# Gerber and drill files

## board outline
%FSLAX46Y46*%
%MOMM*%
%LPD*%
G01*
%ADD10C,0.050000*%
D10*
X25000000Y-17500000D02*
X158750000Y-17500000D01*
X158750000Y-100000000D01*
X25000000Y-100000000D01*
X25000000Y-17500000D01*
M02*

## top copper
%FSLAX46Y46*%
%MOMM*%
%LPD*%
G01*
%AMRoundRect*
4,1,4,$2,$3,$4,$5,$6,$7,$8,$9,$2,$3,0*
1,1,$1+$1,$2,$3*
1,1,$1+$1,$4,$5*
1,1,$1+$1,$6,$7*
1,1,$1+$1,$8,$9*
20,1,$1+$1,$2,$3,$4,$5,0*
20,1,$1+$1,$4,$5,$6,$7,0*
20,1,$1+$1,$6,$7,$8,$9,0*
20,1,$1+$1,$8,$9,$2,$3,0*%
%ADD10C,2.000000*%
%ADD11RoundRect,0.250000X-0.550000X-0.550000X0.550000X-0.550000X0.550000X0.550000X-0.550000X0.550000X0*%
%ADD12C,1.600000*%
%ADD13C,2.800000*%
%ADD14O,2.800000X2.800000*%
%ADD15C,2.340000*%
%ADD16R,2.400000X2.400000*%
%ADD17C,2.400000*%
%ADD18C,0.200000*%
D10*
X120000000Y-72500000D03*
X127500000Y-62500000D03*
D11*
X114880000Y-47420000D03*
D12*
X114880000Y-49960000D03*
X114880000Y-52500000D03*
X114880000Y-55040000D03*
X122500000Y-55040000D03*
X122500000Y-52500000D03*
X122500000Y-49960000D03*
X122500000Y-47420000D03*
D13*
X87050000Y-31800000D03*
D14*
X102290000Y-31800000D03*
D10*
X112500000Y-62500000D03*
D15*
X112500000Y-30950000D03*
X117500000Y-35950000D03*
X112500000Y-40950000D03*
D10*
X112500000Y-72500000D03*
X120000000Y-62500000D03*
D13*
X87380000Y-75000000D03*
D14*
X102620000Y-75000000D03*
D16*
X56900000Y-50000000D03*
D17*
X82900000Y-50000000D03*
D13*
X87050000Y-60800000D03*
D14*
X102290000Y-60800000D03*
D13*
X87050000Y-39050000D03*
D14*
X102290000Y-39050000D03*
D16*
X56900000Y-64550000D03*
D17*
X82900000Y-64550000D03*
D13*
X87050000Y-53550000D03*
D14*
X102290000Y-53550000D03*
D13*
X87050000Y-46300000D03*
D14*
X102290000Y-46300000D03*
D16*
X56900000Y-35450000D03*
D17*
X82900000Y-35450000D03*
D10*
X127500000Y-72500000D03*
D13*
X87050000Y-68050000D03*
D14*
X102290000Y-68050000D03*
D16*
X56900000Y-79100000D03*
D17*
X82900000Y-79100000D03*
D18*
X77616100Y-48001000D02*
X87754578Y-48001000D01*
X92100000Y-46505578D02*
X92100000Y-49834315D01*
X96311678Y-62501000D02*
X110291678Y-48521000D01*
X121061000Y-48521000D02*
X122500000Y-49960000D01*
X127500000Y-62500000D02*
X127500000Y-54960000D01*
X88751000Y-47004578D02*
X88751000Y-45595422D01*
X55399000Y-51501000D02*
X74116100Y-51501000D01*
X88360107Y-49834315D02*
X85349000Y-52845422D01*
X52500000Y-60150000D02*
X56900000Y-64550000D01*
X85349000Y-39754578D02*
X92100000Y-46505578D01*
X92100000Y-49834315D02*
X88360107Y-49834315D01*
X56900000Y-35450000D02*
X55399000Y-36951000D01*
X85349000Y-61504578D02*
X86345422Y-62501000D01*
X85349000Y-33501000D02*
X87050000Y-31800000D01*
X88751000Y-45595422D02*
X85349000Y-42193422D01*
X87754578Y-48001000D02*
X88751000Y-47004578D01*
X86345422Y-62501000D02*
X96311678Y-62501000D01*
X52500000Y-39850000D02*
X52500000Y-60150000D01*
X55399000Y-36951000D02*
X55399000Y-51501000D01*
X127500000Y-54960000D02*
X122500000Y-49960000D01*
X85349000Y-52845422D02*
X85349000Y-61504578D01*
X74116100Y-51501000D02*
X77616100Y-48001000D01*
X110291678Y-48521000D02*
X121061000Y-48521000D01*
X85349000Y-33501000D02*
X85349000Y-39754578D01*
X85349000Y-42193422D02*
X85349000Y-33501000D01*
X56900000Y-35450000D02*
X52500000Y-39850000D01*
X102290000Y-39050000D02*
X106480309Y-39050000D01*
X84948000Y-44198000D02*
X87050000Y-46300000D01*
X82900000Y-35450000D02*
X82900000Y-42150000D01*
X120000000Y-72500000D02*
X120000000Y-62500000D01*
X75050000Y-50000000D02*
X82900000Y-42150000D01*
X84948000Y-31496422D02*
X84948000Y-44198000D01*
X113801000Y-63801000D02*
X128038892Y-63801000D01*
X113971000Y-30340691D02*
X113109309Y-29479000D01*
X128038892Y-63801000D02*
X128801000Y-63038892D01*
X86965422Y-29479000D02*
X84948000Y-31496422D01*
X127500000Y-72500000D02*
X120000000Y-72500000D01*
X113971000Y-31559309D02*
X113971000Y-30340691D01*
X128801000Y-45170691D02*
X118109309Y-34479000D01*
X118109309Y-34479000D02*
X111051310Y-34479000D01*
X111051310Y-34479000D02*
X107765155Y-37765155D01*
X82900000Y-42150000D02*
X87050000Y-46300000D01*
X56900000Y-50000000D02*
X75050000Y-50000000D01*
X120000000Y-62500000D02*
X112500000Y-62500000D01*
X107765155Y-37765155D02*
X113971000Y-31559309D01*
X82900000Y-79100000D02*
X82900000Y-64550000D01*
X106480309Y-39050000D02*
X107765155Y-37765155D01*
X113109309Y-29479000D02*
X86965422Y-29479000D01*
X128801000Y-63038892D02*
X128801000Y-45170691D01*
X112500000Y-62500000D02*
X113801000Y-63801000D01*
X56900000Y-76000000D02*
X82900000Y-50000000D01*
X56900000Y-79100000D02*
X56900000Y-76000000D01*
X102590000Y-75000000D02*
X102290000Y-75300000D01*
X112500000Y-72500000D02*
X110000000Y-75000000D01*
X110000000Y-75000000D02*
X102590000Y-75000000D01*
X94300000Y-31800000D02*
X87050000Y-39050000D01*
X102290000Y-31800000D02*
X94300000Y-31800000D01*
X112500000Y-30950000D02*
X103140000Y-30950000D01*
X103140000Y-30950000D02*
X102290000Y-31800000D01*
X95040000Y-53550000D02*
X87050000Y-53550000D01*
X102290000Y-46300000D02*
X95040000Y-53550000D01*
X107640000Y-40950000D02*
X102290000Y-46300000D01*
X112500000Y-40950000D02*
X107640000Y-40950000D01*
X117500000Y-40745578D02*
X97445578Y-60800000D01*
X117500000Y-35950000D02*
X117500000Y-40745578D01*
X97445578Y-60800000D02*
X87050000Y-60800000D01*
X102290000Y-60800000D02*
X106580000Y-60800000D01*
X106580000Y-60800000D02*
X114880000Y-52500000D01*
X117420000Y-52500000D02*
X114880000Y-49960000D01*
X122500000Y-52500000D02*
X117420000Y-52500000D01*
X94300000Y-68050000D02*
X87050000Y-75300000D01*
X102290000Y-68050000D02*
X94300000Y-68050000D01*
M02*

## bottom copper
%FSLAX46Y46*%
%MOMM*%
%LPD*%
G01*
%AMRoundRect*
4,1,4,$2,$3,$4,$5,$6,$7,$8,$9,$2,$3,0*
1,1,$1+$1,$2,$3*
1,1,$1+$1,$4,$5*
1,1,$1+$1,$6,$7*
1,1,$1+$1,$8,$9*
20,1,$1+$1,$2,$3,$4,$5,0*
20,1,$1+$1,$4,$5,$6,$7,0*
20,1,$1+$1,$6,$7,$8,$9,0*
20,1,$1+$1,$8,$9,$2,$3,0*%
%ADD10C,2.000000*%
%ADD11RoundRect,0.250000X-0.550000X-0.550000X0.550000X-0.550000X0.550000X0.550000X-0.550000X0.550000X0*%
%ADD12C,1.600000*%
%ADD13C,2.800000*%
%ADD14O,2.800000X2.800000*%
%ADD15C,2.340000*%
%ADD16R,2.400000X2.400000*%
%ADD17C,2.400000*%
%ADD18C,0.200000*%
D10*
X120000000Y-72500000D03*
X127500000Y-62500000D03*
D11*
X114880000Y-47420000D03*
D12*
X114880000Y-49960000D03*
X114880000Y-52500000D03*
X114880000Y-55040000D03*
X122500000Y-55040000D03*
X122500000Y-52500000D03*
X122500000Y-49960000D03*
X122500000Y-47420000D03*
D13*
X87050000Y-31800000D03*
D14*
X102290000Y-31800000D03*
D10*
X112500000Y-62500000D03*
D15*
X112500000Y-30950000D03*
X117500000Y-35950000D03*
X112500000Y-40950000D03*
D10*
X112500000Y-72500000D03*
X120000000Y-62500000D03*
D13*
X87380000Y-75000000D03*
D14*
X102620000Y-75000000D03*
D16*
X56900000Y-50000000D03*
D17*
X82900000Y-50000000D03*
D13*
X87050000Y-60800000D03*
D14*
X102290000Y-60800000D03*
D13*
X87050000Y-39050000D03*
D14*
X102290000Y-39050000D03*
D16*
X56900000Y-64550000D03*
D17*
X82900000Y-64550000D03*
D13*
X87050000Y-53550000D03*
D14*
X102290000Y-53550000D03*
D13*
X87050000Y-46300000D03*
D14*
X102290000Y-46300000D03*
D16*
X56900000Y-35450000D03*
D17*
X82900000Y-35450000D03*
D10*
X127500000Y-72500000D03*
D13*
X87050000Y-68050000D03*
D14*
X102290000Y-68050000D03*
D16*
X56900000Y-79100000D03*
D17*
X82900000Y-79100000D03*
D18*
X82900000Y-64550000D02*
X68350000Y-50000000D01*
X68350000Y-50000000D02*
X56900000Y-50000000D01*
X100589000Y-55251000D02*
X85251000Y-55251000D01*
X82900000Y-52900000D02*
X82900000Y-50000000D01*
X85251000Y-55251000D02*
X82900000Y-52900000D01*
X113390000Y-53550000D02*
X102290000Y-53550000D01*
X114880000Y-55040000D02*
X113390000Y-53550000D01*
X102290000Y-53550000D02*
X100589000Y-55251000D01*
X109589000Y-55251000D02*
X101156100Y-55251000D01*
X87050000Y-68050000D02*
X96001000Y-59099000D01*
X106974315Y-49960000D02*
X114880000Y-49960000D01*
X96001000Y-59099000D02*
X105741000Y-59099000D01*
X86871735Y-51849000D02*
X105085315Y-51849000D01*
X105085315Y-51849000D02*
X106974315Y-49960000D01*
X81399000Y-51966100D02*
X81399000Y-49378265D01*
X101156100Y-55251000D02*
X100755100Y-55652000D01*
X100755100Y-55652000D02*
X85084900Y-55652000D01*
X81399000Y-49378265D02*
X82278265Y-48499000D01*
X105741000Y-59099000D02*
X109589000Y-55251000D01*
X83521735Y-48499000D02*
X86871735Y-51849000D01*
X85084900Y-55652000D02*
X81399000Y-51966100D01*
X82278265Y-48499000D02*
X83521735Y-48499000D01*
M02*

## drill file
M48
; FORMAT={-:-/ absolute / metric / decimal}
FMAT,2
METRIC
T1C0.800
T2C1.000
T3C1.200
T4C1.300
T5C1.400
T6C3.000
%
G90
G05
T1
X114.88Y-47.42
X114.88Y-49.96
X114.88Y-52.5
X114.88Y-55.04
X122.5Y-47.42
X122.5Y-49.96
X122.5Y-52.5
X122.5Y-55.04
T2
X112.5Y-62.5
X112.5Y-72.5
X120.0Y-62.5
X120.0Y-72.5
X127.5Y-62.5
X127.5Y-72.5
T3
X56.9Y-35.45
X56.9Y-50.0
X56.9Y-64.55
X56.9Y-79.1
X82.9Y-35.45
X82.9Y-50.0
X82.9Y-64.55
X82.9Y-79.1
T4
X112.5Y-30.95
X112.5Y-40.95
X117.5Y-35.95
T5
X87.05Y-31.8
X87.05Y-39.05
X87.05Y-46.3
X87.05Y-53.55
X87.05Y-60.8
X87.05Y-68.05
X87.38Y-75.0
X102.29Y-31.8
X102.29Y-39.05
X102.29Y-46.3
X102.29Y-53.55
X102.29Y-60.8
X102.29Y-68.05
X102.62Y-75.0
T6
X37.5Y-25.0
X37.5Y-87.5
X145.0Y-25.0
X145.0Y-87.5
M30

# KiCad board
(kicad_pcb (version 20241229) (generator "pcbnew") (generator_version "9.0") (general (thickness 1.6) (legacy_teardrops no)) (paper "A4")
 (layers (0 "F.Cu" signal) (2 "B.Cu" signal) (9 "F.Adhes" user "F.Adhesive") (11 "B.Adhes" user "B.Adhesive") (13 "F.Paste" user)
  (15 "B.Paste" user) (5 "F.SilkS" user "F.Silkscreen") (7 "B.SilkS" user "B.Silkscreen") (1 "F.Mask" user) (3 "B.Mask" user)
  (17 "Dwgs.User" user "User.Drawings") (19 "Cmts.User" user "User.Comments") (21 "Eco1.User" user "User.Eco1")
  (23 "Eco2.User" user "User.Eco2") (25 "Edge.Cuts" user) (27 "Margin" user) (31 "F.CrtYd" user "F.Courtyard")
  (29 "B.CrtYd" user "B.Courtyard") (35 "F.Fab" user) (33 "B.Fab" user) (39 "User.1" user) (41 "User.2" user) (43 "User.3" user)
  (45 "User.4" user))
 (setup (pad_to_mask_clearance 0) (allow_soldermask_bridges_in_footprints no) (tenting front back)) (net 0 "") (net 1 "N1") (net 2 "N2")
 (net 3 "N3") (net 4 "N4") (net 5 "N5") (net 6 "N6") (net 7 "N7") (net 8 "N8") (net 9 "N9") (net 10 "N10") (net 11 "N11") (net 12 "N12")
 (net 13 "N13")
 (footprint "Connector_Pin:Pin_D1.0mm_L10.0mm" (layer "F.Cu") (at 120 72.5)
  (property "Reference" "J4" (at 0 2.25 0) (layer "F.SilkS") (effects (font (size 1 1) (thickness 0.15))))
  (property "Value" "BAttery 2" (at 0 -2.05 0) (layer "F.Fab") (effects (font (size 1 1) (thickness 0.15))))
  (pad "1" thru_hole circle (at 0 0) (size 2 2) (drill 1) (layers "*.Cu" "*.Mask") (remove_unused_layers no) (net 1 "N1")))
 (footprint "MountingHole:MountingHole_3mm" (layer "F.Cu") (at 145 25)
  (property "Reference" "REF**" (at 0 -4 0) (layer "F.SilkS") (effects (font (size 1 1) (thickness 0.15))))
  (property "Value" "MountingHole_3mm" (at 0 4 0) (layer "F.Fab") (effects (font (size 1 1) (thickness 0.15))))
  (pad "" np_thru_hole circle (at 0 0) (size 3 3) (drill 3) (layers "*.Cu" "*.Mask")))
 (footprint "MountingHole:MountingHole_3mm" (layer "F.Cu") (at 37.5 25)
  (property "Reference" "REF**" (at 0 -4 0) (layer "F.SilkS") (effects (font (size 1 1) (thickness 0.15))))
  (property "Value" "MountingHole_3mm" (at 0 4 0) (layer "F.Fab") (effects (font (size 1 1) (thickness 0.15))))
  (pad "" np_thru_hole circle (at 0 0) (size 3 3) (drill 3) (layers "*.Cu" "*.Mask")))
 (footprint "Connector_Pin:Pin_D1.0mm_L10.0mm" (layer "F.Cu") (at 127.5 62.5)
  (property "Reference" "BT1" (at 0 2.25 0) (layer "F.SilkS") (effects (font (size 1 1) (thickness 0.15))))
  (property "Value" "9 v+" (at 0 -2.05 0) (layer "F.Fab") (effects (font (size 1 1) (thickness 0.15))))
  (pad "1" thru_hole circle (at 0 0) (size 2 2) (drill 1) (layers "*.Cu" "*.Mask") (remove_unused_layers no) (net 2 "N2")))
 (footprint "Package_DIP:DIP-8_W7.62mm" (layer "F.Cu") (at 114.88 47.42)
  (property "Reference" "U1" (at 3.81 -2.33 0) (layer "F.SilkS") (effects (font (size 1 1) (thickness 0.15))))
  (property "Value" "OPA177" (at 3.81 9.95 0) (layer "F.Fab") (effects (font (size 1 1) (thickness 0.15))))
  (pad "1" thru_hole roundrect (at 0 0) (size 1.6 1.6) (drill 0.8) (layers "*.Cu" "*.Mask") (remove_unused_layers no)
   (roundrect_rratio 0.15625) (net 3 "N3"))
  (pad "2" thru_hole circle (at 0 2.54) (size 1.6 1.6) (drill 0.8) (layers "*.Cu" "*.Mask") (remove_unused_layers no) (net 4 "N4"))
  (pad "3" thru_hole circle (at 0 5.08) (size 1.6 1.6) (drill 0.8) (layers "*.Cu" "*.Mask") (remove_unused_layers no) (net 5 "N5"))
  (pad "4" thru_hole circle (at 0 7.62) (size 1.6 1.6) (drill 0.8) (layers "*.Cu" "*.Mask") (remove_unused_layers no) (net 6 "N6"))
  (pad "5" thru_hole circle (at 7.62 7.62) (size 1.6 1.6) (drill 0.8) (layers "*.Cu" "*.Mask") (remove_unused_layers no) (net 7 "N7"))
  (pad "6" thru_hole circle (at 7.62 5.08) (size 1.6 1.6) (drill 0.8) (layers "*.Cu" "*.Mask") (remove_unused_layers no) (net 4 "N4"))
  (pad "7" thru_hole circle (at 7.62 2.54) (size 1.6 1.6) (drill 0.8) (layers "*.Cu" "*.Mask") (remove_unused_layers no) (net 2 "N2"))
  (pad "8" thru_hole circle (at 7.62 0) (size 1.6 1.6) (drill 0.8) (layers "*.Cu" "*.Mask") (remove_unused_layers no) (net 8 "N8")))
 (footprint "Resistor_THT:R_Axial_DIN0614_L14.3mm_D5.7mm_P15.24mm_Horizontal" (layer "F.Cu") (at 87.05 31.8)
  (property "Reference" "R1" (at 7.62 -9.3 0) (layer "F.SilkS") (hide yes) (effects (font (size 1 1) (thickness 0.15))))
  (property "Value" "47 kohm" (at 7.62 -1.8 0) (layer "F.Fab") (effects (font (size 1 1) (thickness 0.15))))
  (pad "1" thru_hole circle (at 0 0) (size 2.8 2.8) (drill 1.4) (layers "*.Cu" "*.Mask") (remove_unused_layers no) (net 2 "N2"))
  (pad "2" thru_hole oval (at 15.24 0) (size 2.8 2.8) (drill 1.4) (layers "*.Cu" "*.Mask") (remove_unused_layers no) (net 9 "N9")))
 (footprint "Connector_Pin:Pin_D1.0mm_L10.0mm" (layer "F.Cu") (at 112.5 62.5)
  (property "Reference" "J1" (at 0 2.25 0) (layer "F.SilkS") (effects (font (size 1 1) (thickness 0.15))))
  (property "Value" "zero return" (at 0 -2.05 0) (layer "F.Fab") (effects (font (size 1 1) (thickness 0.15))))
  (pad "1" thru_hole circle (at 0 0) (size 2 2) (drill 1) (layers "*.Cu" "*.Mask") (remove_unused_layers no) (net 1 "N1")))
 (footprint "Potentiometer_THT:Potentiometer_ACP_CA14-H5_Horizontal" (layer "F.Cu") (at 112.5 30.95)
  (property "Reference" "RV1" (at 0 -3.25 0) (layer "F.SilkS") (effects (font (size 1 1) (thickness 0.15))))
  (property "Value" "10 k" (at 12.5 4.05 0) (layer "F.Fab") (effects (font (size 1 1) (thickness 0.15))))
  (pad "1" thru_hole circle (at 0 0) (size 2.34 2.34) (drill 1.3) (layers "*.Cu" "*.Mask") (remove_unused_layers no) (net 9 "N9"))
  (pad "2" thru_hole circle (at 5 5) (size 2.34 2.34) (drill 1.3) (layers "*.Cu" "*.Mask") (remove_unused_layers no) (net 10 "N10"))
  (pad "3" thru_hole circle (at 0 10) (size 2.34 2.34) (drill 1.3) (layers "*.Cu" "*.Mask") (remove_unused_layers no) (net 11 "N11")))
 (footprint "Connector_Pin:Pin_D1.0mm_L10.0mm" (layer "F.Cu") (at 112.5 72.5)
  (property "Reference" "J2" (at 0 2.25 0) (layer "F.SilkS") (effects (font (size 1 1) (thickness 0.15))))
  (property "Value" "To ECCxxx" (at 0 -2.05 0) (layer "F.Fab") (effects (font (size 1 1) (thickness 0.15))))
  (pad "1" thru_hole circle (at 0 0) (size 2 2) (drill 1) (layers "*.Cu" "*.Mask") (remove_unused_layers no) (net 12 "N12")))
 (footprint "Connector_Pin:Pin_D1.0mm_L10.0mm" (layer "F.Cu") (at 120 62.5)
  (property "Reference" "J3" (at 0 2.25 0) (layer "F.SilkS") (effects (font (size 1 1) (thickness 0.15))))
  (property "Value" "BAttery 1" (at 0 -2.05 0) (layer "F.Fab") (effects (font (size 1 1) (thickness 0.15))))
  (pad "1" thru_hole circle (at 0 0) (size 2 2) (drill 1) (layers "*.Cu" "*.Mask") (remove_unused_layers no) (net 1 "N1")))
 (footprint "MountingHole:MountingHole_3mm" (layer "F.Cu") (at 37.5 87.5)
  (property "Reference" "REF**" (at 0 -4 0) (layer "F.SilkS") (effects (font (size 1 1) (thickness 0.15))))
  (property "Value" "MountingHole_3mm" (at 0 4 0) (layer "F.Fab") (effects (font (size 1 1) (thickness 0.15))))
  (pad "" np_thru_hole circle (at 0 0) (size 3 3) (drill 3) (layers "*.Cu" "*.Mask")))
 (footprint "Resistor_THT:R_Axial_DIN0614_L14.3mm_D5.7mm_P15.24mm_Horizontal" (layer "F.Cu") (at 87.38 75)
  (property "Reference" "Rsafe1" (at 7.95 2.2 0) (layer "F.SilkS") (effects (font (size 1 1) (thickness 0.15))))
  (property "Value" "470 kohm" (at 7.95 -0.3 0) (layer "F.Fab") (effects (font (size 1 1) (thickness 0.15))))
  (pad "1" thru_hole circle (at 0 0) (size 2.8 2.8) (drill 1.4) (layers "*.Cu" "*.Mask") (remove_unused_layers no) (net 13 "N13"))
  (pad "2" thru_hole oval (at 15.24 0) (size 2.8 2.8) (drill 1.4) (layers "*.Cu" "*.Mask") (remove_unused_layers no) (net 12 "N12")))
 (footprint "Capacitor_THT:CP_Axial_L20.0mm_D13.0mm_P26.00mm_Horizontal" (layer "F.Cu") (at 56.9 50)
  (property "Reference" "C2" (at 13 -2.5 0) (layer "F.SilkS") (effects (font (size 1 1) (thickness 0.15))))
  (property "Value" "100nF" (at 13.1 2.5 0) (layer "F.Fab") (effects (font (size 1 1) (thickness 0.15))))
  (pad "1" thru_hole rect (at 0 0) (size 2.4 2.4) (drill 1.2) (layers "*.Cu" "*.Mask") (remove_unused_layers no) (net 1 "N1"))
  (pad "2" thru_hole circle (at 26 0) (size 2.4 2.4) (drill 1.2) (layers "*.Cu" "*.Mask") (remove_unused_layers no) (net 6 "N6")))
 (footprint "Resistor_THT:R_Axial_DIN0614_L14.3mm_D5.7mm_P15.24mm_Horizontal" (layer "F.Cu") (at 87.05 60.8)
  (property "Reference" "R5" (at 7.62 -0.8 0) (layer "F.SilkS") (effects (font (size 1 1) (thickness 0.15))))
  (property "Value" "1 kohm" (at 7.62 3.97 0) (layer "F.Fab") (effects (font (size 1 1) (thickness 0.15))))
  (pad "1" thru_hole circle (at 0 0) (size 2.8 2.8) (drill 1.4) (layers "*.Cu" "*.Mask") (remove_unused_layers no) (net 10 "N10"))
  (pad "2" thru_hole oval (at 15.24 0) (size 2.8 2.8) (drill 1.4) (layers "*.Cu" "*.Mask") (remove_unused_layers no) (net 5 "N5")))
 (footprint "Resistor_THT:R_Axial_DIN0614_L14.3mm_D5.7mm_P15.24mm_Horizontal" (layer "F.Cu") (at 87.05 39.05)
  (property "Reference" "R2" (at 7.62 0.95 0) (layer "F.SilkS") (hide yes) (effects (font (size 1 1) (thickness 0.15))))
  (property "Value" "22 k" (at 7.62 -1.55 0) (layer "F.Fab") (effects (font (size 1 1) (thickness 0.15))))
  (pad "1" thru_hole circle (at 0 0) (size 2.8 2.8) (drill 1.4) (layers "*.Cu" "*.Mask") (remove_unused_layers no) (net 9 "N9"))
  (pad "2" thru_hole oval (at 15.24 0) (size 2.8 2.8) (drill 1.4) (layers "*.Cu" "*.Mask") (remove_unused_layers no) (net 1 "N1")))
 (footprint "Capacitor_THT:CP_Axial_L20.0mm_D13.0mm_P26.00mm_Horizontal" (layer "F.Cu") (at 56.9 64.55)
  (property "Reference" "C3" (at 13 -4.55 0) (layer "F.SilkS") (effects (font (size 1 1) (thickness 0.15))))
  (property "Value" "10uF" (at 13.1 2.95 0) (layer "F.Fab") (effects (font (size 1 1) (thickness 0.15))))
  (pad "1" thru_hole rect (at 0 0) (size 2.4 2.4) (drill 1.2) (layers "*.Cu" "*.Mask") (remove_unused_layers no) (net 2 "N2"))
  (pad "2" thru_hole circle (at 26 0) (size 2.4 2.4) (drill 1.2) (layers "*.Cu" "*.Mask") (remove_unused_layers no) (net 1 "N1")))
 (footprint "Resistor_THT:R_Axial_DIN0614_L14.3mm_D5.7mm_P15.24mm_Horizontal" (layer "F.Cu") (at 87.05 53.55)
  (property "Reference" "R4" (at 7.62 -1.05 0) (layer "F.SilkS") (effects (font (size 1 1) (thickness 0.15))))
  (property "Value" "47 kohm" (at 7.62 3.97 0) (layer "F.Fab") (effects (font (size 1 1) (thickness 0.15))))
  (pad "1" thru_hole circle (at 0 0) (size 2.8 2.8) (drill 1.4) (layers "*.Cu" "*.Mask") (remove_unused_layers no) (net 11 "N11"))
  (pad "2" thru_hole oval (at 15.24 0) (size 2.8 2.8) (drill 1.4) (layers "*.Cu" "*.Mask") (remove_unused_layers no) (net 6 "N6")))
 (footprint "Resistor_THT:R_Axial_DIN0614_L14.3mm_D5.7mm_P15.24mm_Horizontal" (layer "F.Cu") (at 87.05 46.3)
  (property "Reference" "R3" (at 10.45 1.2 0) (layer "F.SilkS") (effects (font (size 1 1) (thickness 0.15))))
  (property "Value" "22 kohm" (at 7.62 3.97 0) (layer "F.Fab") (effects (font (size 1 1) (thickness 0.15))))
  (pad "1" thru_hole circle (at 0 0) (size 2.8 2.8) (drill 1.4) (layers "*.Cu" "*.Mask") (remove_unused_layers no) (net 1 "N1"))
  (pad "2" thru_hole oval (at 15.24 0) (size 2.8 2.8) (drill 1.4) (layers "*.Cu" "*.Mask") (remove_unused_layers no) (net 11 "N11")))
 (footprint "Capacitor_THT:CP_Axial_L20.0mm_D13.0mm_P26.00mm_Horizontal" (layer "F.Cu") (at 56.9 35.45)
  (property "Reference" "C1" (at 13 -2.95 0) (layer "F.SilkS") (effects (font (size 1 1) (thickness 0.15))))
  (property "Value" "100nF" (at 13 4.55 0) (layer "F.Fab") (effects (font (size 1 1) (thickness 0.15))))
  (pad "1" thru_hole rect (at 0 0) (size 2.4 2.4) (drill 1.2) (layers "*.Cu" "*.Mask") (remove_unused_layers no) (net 2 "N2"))
  (pad "2" thru_hole circle (at 26 0) (size 2.4 2.4) (drill 1.2) (layers "*.Cu" "*.Mask") (remove_unused_layers no) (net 1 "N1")))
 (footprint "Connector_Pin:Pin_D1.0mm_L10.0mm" (layer "F.Cu") (at 127.5 72.5)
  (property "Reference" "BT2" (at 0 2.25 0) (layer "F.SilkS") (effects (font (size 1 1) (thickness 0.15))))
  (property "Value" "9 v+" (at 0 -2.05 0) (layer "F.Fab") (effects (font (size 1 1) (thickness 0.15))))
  (pad "1" thru_hole circle (at 0 0) (size 2 2) (drill 1) (layers "*.Cu" "*.Mask") (remove_unused_layers no) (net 1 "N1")))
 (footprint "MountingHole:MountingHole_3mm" (layer "F.Cu") (at 145 87.5)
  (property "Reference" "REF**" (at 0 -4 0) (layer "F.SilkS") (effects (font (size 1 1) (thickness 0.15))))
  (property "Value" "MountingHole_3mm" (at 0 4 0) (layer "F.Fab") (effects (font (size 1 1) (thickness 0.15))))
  (pad "" np_thru_hole circle (at 0 0) (size 3 3) (drill 3) (layers "*.Cu" "*.Mask")))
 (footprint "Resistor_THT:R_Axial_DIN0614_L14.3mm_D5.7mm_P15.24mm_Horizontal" (layer "F.Cu") (at 87.05 68.05)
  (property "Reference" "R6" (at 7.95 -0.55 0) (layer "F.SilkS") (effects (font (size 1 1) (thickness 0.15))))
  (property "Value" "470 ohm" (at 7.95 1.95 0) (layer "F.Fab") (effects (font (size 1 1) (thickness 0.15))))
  (pad "1" thru_hole circle (at 0 0) (size 2.8 2.8) (drill 1.4) (layers "*.Cu" "*.Mask") (remove_unused_layers no) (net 4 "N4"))
  (pad "2" thru_hole oval (at 15.24 0) (size 2.8 2.8) (drill 1.4) (layers "*.Cu" "*.Mask") (remove_unused_layers no) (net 13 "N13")))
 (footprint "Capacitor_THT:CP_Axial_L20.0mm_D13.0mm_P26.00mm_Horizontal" (layer "F.Cu") (at 56.9 79.1)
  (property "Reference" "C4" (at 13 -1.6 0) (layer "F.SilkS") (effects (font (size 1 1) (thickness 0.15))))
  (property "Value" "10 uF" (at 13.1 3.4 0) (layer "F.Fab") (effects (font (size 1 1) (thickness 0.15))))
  (pad "1" thru_hole rect (at 0 0) (size 2.4 2.4) (drill 1.2) (layers "*.Cu" "*.Mask") (remove_unused_layers no) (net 6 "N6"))
  (pad "2" thru_hole circle (at 26 0) (size 2.4 2.4) (drill 1.2) (layers "*.Cu" "*.Mask") (remove_unused_layers no) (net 1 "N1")))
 (gr_rect (start 25 17.5) (end 158.75 100) (stroke (width 0.05) (type default)) (fill no) (layer "Edge.Cuts"))
 (segment (start 77.6161 48.001) (end 87.754578 48.001) (width 0.2) (layer "F.Cu") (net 2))
 (segment (start 92.1 46.505578) (end 92.1 49.834315) (width 0.2) (layer "F.Cu") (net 2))
 (segment (start 96.311678 62.501) (end 110.291678 48.521) (width 0.2) (layer "F.Cu") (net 2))
 (segment (start 121.061 48.521) (end 122.5 49.96) (width 0.2) (layer "F.Cu") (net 2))
 (segment (start 127.5 62.5) (end 127.5 54.96) (width 0.2) (layer "F.Cu") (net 2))
 (segment (start 88.751 47.004578) (end 88.751 45.595422) (width 0.2) (layer "F.Cu") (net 2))
 (segment (start 55.399 51.501) (end 74.1161 51.501) (width 0.2) (layer "F.Cu") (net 2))
 (segment (start 88.360107 49.834315) (end 85.349 52.845422) (width 0.2) (layer "F.Cu") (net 2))
 (segment (start 52.5 60.15) (end 56.9 64.55) (width 0.2) (layer "F.Cu") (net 2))
 (segment (start 85.349 39.754578) (end 92.1 46.505578) (width 0.2) (layer "F.Cu") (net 2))
 (segment (start 92.1 49.834315) (end 88.360107 49.834315) (width 0.2) (layer "F.Cu") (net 2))
 (segment (start 56.9 35.45) (end 55.399 36.951) (width 0.2) (layer "F.Cu") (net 2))
 (segment (start 85.349 61.504578) (end 86.345422 62.501) (width 0.2) (layer "F.Cu") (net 2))
 (segment (start 85.349 33.501) (end 87.05 31.8) (width 0.2) (layer "F.Cu") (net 2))
 (segment (start 88.751 45.595422) (end 85.349 42.193422) (width 0.2) (layer "F.Cu") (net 2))
 (segment (start 87.754578 48.001) (end 88.751 47.004578) (width 0.2) (layer "F.Cu") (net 2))
 (segment (start 86.345422 62.501) (end 96.311678 62.501) (width 0.2) (layer "F.Cu") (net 2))
 (segment (start 52.5 39.85) (end 52.5 60.15) (width 0.2) (layer "F.Cu") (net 2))
 (segment (start 55.399 36.951) (end 55.399 51.501) (width 0.2) (layer "F.Cu") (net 2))
 (segment (start 127.5 54.96) (end 122.5 49.96) (width 0.2) (layer "F.Cu") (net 2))
 (segment (start 85.349 52.845422) (end 85.349 61.504578) (width 0.2) (layer "F.Cu") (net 2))
 (segment (start 74.1161 51.501) (end 77.6161 48.001) (width 0.2) (layer "F.Cu") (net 2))
 (segment (start 110.291678 48.521) (end 121.061 48.521) (width 0.2) (layer "F.Cu") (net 2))
 (segment (start 85.349 33.501) (end 85.349 39.754578) (width 0.2) (layer "F.Cu") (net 2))
 (segment (start 85.349 42.193422) (end 85.349 33.501) (width 0.2) (layer "F.Cu") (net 2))
 (segment (start 56.9 35.45) (end 52.5 39.85) (width 0.2) (layer "F.Cu") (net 2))
 (segment (start 102.29 39.05) (end 106.480309 39.05) (width 0.2) (layer "F.Cu") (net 1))
 (segment (start 84.948 44.198) (end 87.05 46.3) (width 0.2) (layer "F.Cu") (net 1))
 (segment (start 82.9 35.45) (end 82.9 42.15) (width 0.2) (layer "F.Cu") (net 1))
 (segment (start 120 72.5) (end 120 62.5) (width 0.2) (layer "F.Cu") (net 1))
 (segment (start 75.05 50) (end 82.9 42.15) (width 0.2) (layer "F.Cu") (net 1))
 (segment (start 84.948 31.496422) (end 84.948 44.198) (width 0.2) (layer "F.Cu") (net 1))
 (segment (start 113.801 63.801) (end 128.038892 63.801) (width 0.2) (layer "F.Cu") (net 1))
 (segment (start 113.971 30.340691) (end 113.109309 29.479) (width 0.2) (layer "F.Cu") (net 1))
 (segment (start 128.038892 63.801) (end 128.801 63.038892) (width 0.2) (layer "F.Cu") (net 1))
 (segment (start 86.965422 29.479) (end 84.948 31.496422) (width 0.2) (layer "F.Cu") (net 1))
 (segment (start 127.5 72.5) (end 120 72.5) (width 0.2) (layer "F.Cu") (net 1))
 (segment (start 113.971 31.559309) (end 113.971 30.340691) (width 0.2) (layer "F.Cu") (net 1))
 (segment (start 128.801 45.170691) (end 118.109309 34.479) (width 0.2) (layer "F.Cu") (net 1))
 (segment (start 118.109309 34.479) (end 111.05131 34.479) (width 0.2) (layer "F.Cu") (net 1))
 (segment (start 111.05131 34.479) (end 107.765155 37.765155) (width 0.2) (layer "F.Cu") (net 1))
 (segment (start 82.9 42.15) (end 87.05 46.3) (width 0.2) (layer "F.Cu") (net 1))
 (segment (start 56.9 50) (end 75.05 50) (width 0.2) (layer "F.Cu") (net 1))
 (segment (start 120 62.5) (end 112.5 62.5) (width 0.2) (layer "F.Cu") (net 1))
 (segment (start 107.765155 37.765155) (end 113.971 31.559309) (width 0.2) (layer "F.Cu") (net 1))
 (segment (start 82.9 79.1) (end 82.9 64.55) (width 0.2) (layer "F.Cu") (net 1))
 (segment (start 106.480309 39.05) (end 107.765155 37.765155) (width 0.2) (layer "F.Cu") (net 1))
 (segment (start 113.109309 29.479) (end 86.965422 29.479) (width 0.2) (layer "F.Cu") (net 1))
 (segment (start 128.801 63.038892) (end 128.801 45.170691) (width 0.2) (layer "F.Cu") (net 1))
 (segment (start 112.5 62.5) (end 113.801 63.801) (width 0.2) (layer "F.Cu") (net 1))
 (segment (start 82.9 64.55) (end 68.35 50) (width 0.2) (layer "B.Cu") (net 1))
 (segment (start 68.35 50) (end 56.9 50) (width 0.2) (layer "B.Cu") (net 1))
 (segment (start 56.9 76) (end 82.9 50) (width 0.2) (layer "F.Cu") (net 6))
 (segment (start 56.9 79.1) (end 56.9 76) (width 0.2) (layer "F.Cu") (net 6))
 (segment (start 100.589 55.251) (end 85.251 55.251) (width 0.2) (layer "B.Cu") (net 6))
 (segment (start 82.9 52.9) (end 82.9 50) (width 0.2) (layer "B.Cu") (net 6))
 (segment (start 85.251 55.251) (end 82.9 52.9) (width 0.2) (layer "B.Cu") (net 6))
 (segment (start 113.39 53.55) (end 102.29 53.55) (width 0.2) (layer "B.Cu") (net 6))
 (segment (start 114.88 55.04) (end 113.39 53.55) (width 0.2) (layer "B.Cu") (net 6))
 (segment (start 102.29 53.55) (end 100.589 55.251) (width 0.2) (layer "B.Cu") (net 6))
 (segment (start 102.59 75) (end 102.29 75.3) (width 0.2) (layer "F.Cu") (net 12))
 (segment (start 112.5 72.5) (end 110 75) (width 0.2) (layer "F.Cu") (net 12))
 (segment (start 110 75) (end 102.59 75) (width 0.2) (layer "F.Cu") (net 12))
 (segment (start 94.3 31.8) (end 87.05 39.05) (width 0.2) (layer "F.Cu") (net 9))
 (segment (start 102.29 31.8) (end 94.3 31.8) (width 0.2) (layer "F.Cu") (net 9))
 (segment (start 112.5 30.95) (end 103.14 30.95) (width 0.2) (layer "F.Cu") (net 9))
 (segment (start 103.14 30.95) (end 102.29 31.8) (width 0.2) (layer "F.Cu") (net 9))
 (segment (start 95.04 53.55) (end 87.05 53.55) (width 0.2) (layer "F.Cu") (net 11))
 (segment (start 102.29 46.3) (end 95.04 53.55) (width 0.2) (layer "F.Cu") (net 11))
 (segment (start 107.64 40.95) (end 102.29 46.3) (width 0.2) (layer "F.Cu") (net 11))
 (segment (start 112.5 40.95) (end 107.64 40.95) (width 0.2) (layer "F.Cu") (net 11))
 (segment (start 117.5 40.745578) (end 97.445578 60.8) (width 0.2) (layer "F.Cu") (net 10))
 (segment (start 117.5 35.95) (end 117.5 40.745578) (width 0.2) (layer "F.Cu") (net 10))
 (segment (start 97.445578 60.8) (end 87.05 60.8) (width 0.2) (layer "F.Cu") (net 10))
 (segment (start 102.29 60.8) (end 106.58 60.8) (width 0.2) (layer "F.Cu") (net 5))
 (segment (start 106.58 60.8) (end 114.88 52.5) (width 0.2) (layer "F.Cu") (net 5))
 (segment (start 117.42 52.5) (end 114.88 49.96) (width 0.2) (layer "F.Cu") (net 4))
 (segment (start 122.5 52.5) (end 117.42 52.5) (width 0.2) (layer "F.Cu") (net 4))
 (segment (start 109.589 55.251) (end 101.1561 55.251) (width 0.2) (layer "B.Cu") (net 4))
 (segment (start 87.05 68.05) (end 96.001 59.099) (width 0.2) (layer "B.Cu") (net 4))
 (segment (start 106.974315 49.96) (end 114.88 49.96) (width 0.2) (layer "B.Cu") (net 4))
 (segment (start 96.001 59.099) (end 105.741 59.099) (width 0.2) (layer "B.Cu") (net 4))
 (segment (start 86.871735 51.849) (end 105.085315 51.849) (width 0.2) (layer "B.Cu") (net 4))
 (segment (start 105.085315 51.849) (end 106.974315 49.96) (width 0.2) (layer "B.Cu") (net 4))
 (segment (start 81.399 51.9661) (end 81.399 49.378265) (width 0.2) (layer "B.Cu") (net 4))
 (segment (start 101.1561 55.251) (end 100.7551 55.652) (width 0.2) (layer "B.Cu") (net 4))
 (segment (start 100.7551 55.652) (end 85.0849 55.652) (width 0.2) (layer "B.Cu") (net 4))
 (segment (start 81.399 49.378265) (end 82.278265 48.499) (width 0.2) (layer "B.Cu") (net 4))
 (segment (start 105.741 59.099) (end 109.589 55.251) (width 0.2) (layer "B.Cu") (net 4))
 (segment (start 83.521735 48.499) (end 86.871735 51.849) (width 0.2) (layer "B.Cu") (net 4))
 (segment (start 85.0849 55.652) (end 81.399 51.9661) (width 0.2) (layer "B.Cu") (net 4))
 (segment (start 82.278265 48.499) (end 83.521735 48.499) (width 0.2) (layer "B.Cu") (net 4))
 (segment (start 94.3 68.05) (end 87.05 75.3) (width 0.2) (layer "F.Cu") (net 13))
 (segment (start 102.29 68.05) (end 94.3 68.05) (width 0.2) (layer "F.Cu") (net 13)))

